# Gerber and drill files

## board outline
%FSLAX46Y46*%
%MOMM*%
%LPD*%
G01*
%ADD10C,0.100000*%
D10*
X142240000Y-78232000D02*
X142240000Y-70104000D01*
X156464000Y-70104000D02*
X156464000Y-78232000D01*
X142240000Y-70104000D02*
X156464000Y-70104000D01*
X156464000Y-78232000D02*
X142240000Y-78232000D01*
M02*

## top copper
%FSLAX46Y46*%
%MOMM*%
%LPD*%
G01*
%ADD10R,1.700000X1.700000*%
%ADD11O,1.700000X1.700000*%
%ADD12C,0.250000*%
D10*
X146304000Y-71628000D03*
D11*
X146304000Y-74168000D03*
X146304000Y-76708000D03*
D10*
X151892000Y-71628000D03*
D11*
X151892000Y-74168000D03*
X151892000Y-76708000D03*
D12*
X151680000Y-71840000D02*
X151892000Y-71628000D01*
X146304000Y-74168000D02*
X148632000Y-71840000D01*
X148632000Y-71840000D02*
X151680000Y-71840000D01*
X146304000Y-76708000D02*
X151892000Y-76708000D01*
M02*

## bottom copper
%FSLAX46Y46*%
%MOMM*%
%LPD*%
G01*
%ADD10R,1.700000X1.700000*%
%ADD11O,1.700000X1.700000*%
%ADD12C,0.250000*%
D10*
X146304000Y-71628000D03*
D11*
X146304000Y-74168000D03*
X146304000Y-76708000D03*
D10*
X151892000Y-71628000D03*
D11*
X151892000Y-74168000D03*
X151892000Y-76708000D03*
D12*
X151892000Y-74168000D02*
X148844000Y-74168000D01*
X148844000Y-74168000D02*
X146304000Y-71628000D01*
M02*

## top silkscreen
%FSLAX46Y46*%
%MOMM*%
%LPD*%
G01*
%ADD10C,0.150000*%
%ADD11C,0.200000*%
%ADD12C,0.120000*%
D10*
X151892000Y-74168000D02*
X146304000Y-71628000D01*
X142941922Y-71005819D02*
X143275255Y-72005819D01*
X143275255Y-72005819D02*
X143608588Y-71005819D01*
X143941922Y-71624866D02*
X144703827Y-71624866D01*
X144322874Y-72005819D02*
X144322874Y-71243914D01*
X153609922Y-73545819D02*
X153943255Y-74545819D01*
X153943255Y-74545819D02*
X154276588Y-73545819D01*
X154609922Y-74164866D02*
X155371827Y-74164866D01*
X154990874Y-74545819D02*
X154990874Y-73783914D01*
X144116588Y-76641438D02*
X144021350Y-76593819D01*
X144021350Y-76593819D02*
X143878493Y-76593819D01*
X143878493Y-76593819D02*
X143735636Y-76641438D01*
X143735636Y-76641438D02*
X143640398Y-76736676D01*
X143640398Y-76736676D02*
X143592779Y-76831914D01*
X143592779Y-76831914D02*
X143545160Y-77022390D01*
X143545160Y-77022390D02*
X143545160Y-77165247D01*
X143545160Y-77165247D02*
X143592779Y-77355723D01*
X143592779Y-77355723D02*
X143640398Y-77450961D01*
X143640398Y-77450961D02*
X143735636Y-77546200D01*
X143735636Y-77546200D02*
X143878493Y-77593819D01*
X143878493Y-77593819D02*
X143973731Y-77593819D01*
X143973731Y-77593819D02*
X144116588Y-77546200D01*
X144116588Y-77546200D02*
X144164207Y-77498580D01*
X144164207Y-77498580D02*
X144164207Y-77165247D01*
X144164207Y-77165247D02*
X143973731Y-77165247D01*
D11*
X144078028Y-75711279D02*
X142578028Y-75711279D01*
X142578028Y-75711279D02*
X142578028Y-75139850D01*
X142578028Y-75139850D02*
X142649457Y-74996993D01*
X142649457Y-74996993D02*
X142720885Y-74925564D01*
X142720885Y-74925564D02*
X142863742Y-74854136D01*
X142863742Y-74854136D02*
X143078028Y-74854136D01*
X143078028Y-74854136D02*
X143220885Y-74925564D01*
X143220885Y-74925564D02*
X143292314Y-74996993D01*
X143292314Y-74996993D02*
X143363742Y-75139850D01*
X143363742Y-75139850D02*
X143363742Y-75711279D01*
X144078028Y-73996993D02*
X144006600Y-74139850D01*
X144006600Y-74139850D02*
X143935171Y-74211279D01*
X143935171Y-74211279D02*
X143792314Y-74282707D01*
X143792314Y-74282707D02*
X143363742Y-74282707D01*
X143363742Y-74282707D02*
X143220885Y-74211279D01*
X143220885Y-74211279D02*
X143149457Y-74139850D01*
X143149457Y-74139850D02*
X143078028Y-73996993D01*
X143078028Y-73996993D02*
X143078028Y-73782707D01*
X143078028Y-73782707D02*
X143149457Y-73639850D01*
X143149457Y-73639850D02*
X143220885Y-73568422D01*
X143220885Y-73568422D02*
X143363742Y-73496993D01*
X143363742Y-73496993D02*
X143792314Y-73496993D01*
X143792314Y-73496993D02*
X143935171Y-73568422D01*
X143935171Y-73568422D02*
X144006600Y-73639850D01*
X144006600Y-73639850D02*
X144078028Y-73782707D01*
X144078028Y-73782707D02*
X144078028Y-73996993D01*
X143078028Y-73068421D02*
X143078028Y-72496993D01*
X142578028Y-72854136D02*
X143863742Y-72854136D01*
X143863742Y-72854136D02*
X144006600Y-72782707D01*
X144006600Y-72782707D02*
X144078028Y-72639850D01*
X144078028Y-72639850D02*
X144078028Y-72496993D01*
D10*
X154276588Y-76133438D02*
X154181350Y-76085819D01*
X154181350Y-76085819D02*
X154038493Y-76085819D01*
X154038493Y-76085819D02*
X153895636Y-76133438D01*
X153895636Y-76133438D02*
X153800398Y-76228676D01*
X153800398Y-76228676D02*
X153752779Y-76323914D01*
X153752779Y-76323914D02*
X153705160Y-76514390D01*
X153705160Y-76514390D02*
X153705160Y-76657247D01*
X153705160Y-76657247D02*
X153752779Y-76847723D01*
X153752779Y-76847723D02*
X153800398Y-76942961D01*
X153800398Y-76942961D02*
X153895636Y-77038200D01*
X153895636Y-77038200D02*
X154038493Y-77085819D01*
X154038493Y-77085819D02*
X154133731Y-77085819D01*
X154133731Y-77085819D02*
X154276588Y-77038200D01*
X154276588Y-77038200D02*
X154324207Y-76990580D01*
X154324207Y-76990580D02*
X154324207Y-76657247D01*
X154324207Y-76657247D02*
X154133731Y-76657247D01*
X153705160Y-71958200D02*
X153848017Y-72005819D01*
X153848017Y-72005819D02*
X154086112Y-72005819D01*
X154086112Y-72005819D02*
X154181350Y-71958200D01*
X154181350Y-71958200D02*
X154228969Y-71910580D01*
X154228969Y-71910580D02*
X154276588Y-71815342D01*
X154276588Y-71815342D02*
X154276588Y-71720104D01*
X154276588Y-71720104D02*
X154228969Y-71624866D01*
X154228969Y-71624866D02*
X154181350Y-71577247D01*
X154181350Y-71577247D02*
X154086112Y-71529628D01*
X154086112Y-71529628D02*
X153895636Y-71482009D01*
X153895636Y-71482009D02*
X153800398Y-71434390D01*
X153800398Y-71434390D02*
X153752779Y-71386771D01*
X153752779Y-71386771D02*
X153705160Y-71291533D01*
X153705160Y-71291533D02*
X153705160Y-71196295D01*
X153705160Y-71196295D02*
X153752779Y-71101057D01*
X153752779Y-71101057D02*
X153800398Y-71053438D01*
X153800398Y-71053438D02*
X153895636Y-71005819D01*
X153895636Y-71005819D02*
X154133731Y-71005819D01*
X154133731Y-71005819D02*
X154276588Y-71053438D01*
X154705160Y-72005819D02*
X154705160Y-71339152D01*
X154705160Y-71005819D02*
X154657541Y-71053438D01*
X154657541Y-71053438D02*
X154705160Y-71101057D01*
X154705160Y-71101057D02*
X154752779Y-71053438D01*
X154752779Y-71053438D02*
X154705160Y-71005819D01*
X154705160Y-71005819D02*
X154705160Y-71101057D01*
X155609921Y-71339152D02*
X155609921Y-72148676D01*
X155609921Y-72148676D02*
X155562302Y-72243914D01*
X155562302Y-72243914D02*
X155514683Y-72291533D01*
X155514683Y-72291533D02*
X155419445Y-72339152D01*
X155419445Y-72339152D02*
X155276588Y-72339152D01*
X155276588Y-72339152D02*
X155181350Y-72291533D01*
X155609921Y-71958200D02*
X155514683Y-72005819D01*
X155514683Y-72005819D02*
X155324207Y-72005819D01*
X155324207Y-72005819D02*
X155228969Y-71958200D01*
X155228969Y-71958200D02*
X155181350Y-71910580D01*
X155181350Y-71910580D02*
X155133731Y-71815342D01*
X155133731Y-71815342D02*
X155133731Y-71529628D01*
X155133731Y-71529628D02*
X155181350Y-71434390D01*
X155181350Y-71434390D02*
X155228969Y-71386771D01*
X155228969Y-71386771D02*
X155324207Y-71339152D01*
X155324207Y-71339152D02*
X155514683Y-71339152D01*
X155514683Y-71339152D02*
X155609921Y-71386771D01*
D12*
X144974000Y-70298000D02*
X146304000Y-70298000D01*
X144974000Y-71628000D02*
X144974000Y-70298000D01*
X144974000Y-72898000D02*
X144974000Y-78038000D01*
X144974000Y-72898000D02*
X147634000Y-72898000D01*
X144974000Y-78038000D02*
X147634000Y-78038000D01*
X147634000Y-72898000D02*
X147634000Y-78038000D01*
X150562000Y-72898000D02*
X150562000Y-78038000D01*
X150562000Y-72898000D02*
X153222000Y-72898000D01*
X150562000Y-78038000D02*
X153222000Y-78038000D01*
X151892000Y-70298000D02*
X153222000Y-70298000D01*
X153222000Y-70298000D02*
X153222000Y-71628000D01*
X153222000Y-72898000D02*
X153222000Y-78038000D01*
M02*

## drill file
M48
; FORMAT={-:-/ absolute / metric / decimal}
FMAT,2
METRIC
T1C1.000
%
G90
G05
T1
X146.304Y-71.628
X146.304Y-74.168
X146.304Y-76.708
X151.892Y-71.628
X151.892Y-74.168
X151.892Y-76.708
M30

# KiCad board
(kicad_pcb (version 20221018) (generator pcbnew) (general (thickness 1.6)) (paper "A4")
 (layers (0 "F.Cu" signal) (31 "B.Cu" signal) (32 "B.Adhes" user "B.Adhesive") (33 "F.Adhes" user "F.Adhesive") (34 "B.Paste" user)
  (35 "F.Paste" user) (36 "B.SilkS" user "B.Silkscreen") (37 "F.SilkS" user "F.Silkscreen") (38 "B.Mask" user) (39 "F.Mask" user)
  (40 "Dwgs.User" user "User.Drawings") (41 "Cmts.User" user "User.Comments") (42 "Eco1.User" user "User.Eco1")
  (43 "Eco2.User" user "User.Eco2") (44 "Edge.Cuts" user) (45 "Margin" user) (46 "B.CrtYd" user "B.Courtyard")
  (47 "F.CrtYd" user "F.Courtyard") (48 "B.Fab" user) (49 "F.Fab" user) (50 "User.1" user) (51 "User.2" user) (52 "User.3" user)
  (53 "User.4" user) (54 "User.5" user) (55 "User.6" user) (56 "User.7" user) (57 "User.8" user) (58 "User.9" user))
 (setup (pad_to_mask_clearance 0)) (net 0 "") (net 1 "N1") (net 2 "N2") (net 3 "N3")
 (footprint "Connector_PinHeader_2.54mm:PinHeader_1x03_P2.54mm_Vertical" (layer "F.Cu") (at 146.304 71.628)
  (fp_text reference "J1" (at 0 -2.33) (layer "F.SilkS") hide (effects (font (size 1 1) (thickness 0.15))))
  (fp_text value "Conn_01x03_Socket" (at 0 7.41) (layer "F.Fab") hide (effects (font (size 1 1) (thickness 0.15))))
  (fp_line (start -1.33 -1.33) (end 0 -1.33) (stroke (width 0.12) (type solid)) (layer "F.SilkS"))
  (fp_line (start -1.33 0) (end -1.33 -1.33) (stroke (width 0.12) (type solid)) (layer "F.SilkS"))
  (fp_line (start -1.33 1.27) (end -1.33 6.41) (stroke (width 0.12) (type solid)) (layer "F.SilkS"))
  (fp_line (start -1.33 1.27) (end 1.33 1.27) (stroke (width 0.12) (type solid)) (layer "F.SilkS"))
  (fp_line (start -1.33 6.41) (end 1.33 6.41) (stroke (width 0.12) (type solid)) (layer "F.SilkS"))
  (fp_line (start 1.33 1.27) (end 1.33 6.41) (stroke (width 0.12) (type solid)) (layer "F.SilkS"))
  (pad "1" thru_hole rect (at 0 0) (size 1.7 1.7) (drill 1) (layers "*.Cu" "*.Mask") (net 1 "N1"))
  (pad "2" thru_hole oval (at 0 2.54) (size 1.7 1.7) (drill 1) (layers "*.Cu" "*.Mask") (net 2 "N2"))
  (pad "3" thru_hole oval (at 0 5.08) (size 1.7 1.7) (drill 1) (layers "*.Cu" "*.Mask") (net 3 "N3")))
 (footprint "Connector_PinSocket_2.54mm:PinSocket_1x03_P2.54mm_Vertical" (layer "F.Cu") (at 151.892 71.628)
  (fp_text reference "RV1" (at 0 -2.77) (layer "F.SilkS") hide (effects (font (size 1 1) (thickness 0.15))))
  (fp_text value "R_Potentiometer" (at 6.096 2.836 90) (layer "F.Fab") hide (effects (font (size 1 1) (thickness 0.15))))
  (fp_line (start -1.33 1.27) (end -1.33 6.41) (stroke (width 0.12) (type solid)) (layer "F.SilkS"))
  (fp_line (start -1.33 1.27) (end 1.33 1.27) (stroke (width 0.12) (type solid)) (layer "F.SilkS"))
  (fp_line (start -1.33 6.41) (end 1.33 6.41) (stroke (width 0.12) (type solid)) (layer "F.SilkS"))
  (fp_line (start 0 -1.33) (end 1.33 -1.33) (stroke (width 0.12) (type solid)) (layer "F.SilkS"))
  (fp_line (start 1.33 -1.33) (end 1.33 0) (stroke (width 0.12) (type solid)) (layer "F.SilkS"))
  (fp_line (start 1.33 1.27) (end 1.33 6.41) (stroke (width 0.12) (type solid)) (layer "F.SilkS"))
  (pad "1" thru_hole rect (at 0 0) (size 1.7 1.7) (drill 1) (layers "*.Cu" "*.Mask") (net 2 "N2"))
  (pad "2" thru_hole oval (at 0 2.54) (size 1.7 1.7) (drill 1) (layers "*.Cu" "*.Mask") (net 1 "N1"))
  (pad "3" thru_hole oval (at 0 5.08) (size 1.7 1.7) (drill 1) (layers "*.Cu" "*.Mask") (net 3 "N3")))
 (gr_line (start 151.892 74.168) (end 146.304 71.628) (stroke (width 0.15) (type default)) (layer "F.SilkS"))
 (gr_line (start 142.24 78.232) (end 142.24 70.104) (stroke (width 0.1) (type default)) (layer "Edge.Cuts"))
 (gr_line (start 156.464 70.104) (end 156.464 78.232) (stroke (width 0.1) (type default)) (layer "Edge.Cuts"))
 (gr_line (start 142.24 70.104) (end 156.464 70.104) (stroke (width 0.1) (type default)) (layer "Edge.Cuts"))
 (gr_line (start 156.464 78.232) (end 142.24 78.232) (stroke (width 0.1) (type default)) (layer "Edge.Cuts"))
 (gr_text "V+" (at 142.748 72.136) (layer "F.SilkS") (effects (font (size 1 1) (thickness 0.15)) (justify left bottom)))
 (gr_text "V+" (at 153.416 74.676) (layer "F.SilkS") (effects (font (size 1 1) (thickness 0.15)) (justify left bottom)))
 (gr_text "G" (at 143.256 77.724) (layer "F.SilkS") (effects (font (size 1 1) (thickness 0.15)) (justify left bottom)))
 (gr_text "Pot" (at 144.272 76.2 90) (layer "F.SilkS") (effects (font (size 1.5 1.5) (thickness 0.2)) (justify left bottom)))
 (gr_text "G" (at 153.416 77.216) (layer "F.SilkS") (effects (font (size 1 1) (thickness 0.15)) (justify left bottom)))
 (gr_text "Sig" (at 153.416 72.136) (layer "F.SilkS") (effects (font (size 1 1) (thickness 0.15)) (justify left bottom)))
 (segment (start 151.892 74.168) (end 148.844 74.168) (width 0.25) (layer "B.Cu") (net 1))
 (segment (start 148.844 74.168) (end 146.304 71.628) (width 0.25) (layer "B.Cu") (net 1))
 (segment (start 151.68 71.84) (end 151.892 71.628) (width 0.25) (layer "F.Cu") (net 2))
 (segment (start 146.304 74.168) (end 148.632 71.84) (width 0.25) (layer "F.Cu") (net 2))
 (segment (start 148.632 71.84) (end 151.68 71.84) (width 0.25) (layer "F.Cu") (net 2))
 (segment (start 146.304 76.708) (end 151.892 76.708) (width 0.25) (layer "F.Cu") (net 3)))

